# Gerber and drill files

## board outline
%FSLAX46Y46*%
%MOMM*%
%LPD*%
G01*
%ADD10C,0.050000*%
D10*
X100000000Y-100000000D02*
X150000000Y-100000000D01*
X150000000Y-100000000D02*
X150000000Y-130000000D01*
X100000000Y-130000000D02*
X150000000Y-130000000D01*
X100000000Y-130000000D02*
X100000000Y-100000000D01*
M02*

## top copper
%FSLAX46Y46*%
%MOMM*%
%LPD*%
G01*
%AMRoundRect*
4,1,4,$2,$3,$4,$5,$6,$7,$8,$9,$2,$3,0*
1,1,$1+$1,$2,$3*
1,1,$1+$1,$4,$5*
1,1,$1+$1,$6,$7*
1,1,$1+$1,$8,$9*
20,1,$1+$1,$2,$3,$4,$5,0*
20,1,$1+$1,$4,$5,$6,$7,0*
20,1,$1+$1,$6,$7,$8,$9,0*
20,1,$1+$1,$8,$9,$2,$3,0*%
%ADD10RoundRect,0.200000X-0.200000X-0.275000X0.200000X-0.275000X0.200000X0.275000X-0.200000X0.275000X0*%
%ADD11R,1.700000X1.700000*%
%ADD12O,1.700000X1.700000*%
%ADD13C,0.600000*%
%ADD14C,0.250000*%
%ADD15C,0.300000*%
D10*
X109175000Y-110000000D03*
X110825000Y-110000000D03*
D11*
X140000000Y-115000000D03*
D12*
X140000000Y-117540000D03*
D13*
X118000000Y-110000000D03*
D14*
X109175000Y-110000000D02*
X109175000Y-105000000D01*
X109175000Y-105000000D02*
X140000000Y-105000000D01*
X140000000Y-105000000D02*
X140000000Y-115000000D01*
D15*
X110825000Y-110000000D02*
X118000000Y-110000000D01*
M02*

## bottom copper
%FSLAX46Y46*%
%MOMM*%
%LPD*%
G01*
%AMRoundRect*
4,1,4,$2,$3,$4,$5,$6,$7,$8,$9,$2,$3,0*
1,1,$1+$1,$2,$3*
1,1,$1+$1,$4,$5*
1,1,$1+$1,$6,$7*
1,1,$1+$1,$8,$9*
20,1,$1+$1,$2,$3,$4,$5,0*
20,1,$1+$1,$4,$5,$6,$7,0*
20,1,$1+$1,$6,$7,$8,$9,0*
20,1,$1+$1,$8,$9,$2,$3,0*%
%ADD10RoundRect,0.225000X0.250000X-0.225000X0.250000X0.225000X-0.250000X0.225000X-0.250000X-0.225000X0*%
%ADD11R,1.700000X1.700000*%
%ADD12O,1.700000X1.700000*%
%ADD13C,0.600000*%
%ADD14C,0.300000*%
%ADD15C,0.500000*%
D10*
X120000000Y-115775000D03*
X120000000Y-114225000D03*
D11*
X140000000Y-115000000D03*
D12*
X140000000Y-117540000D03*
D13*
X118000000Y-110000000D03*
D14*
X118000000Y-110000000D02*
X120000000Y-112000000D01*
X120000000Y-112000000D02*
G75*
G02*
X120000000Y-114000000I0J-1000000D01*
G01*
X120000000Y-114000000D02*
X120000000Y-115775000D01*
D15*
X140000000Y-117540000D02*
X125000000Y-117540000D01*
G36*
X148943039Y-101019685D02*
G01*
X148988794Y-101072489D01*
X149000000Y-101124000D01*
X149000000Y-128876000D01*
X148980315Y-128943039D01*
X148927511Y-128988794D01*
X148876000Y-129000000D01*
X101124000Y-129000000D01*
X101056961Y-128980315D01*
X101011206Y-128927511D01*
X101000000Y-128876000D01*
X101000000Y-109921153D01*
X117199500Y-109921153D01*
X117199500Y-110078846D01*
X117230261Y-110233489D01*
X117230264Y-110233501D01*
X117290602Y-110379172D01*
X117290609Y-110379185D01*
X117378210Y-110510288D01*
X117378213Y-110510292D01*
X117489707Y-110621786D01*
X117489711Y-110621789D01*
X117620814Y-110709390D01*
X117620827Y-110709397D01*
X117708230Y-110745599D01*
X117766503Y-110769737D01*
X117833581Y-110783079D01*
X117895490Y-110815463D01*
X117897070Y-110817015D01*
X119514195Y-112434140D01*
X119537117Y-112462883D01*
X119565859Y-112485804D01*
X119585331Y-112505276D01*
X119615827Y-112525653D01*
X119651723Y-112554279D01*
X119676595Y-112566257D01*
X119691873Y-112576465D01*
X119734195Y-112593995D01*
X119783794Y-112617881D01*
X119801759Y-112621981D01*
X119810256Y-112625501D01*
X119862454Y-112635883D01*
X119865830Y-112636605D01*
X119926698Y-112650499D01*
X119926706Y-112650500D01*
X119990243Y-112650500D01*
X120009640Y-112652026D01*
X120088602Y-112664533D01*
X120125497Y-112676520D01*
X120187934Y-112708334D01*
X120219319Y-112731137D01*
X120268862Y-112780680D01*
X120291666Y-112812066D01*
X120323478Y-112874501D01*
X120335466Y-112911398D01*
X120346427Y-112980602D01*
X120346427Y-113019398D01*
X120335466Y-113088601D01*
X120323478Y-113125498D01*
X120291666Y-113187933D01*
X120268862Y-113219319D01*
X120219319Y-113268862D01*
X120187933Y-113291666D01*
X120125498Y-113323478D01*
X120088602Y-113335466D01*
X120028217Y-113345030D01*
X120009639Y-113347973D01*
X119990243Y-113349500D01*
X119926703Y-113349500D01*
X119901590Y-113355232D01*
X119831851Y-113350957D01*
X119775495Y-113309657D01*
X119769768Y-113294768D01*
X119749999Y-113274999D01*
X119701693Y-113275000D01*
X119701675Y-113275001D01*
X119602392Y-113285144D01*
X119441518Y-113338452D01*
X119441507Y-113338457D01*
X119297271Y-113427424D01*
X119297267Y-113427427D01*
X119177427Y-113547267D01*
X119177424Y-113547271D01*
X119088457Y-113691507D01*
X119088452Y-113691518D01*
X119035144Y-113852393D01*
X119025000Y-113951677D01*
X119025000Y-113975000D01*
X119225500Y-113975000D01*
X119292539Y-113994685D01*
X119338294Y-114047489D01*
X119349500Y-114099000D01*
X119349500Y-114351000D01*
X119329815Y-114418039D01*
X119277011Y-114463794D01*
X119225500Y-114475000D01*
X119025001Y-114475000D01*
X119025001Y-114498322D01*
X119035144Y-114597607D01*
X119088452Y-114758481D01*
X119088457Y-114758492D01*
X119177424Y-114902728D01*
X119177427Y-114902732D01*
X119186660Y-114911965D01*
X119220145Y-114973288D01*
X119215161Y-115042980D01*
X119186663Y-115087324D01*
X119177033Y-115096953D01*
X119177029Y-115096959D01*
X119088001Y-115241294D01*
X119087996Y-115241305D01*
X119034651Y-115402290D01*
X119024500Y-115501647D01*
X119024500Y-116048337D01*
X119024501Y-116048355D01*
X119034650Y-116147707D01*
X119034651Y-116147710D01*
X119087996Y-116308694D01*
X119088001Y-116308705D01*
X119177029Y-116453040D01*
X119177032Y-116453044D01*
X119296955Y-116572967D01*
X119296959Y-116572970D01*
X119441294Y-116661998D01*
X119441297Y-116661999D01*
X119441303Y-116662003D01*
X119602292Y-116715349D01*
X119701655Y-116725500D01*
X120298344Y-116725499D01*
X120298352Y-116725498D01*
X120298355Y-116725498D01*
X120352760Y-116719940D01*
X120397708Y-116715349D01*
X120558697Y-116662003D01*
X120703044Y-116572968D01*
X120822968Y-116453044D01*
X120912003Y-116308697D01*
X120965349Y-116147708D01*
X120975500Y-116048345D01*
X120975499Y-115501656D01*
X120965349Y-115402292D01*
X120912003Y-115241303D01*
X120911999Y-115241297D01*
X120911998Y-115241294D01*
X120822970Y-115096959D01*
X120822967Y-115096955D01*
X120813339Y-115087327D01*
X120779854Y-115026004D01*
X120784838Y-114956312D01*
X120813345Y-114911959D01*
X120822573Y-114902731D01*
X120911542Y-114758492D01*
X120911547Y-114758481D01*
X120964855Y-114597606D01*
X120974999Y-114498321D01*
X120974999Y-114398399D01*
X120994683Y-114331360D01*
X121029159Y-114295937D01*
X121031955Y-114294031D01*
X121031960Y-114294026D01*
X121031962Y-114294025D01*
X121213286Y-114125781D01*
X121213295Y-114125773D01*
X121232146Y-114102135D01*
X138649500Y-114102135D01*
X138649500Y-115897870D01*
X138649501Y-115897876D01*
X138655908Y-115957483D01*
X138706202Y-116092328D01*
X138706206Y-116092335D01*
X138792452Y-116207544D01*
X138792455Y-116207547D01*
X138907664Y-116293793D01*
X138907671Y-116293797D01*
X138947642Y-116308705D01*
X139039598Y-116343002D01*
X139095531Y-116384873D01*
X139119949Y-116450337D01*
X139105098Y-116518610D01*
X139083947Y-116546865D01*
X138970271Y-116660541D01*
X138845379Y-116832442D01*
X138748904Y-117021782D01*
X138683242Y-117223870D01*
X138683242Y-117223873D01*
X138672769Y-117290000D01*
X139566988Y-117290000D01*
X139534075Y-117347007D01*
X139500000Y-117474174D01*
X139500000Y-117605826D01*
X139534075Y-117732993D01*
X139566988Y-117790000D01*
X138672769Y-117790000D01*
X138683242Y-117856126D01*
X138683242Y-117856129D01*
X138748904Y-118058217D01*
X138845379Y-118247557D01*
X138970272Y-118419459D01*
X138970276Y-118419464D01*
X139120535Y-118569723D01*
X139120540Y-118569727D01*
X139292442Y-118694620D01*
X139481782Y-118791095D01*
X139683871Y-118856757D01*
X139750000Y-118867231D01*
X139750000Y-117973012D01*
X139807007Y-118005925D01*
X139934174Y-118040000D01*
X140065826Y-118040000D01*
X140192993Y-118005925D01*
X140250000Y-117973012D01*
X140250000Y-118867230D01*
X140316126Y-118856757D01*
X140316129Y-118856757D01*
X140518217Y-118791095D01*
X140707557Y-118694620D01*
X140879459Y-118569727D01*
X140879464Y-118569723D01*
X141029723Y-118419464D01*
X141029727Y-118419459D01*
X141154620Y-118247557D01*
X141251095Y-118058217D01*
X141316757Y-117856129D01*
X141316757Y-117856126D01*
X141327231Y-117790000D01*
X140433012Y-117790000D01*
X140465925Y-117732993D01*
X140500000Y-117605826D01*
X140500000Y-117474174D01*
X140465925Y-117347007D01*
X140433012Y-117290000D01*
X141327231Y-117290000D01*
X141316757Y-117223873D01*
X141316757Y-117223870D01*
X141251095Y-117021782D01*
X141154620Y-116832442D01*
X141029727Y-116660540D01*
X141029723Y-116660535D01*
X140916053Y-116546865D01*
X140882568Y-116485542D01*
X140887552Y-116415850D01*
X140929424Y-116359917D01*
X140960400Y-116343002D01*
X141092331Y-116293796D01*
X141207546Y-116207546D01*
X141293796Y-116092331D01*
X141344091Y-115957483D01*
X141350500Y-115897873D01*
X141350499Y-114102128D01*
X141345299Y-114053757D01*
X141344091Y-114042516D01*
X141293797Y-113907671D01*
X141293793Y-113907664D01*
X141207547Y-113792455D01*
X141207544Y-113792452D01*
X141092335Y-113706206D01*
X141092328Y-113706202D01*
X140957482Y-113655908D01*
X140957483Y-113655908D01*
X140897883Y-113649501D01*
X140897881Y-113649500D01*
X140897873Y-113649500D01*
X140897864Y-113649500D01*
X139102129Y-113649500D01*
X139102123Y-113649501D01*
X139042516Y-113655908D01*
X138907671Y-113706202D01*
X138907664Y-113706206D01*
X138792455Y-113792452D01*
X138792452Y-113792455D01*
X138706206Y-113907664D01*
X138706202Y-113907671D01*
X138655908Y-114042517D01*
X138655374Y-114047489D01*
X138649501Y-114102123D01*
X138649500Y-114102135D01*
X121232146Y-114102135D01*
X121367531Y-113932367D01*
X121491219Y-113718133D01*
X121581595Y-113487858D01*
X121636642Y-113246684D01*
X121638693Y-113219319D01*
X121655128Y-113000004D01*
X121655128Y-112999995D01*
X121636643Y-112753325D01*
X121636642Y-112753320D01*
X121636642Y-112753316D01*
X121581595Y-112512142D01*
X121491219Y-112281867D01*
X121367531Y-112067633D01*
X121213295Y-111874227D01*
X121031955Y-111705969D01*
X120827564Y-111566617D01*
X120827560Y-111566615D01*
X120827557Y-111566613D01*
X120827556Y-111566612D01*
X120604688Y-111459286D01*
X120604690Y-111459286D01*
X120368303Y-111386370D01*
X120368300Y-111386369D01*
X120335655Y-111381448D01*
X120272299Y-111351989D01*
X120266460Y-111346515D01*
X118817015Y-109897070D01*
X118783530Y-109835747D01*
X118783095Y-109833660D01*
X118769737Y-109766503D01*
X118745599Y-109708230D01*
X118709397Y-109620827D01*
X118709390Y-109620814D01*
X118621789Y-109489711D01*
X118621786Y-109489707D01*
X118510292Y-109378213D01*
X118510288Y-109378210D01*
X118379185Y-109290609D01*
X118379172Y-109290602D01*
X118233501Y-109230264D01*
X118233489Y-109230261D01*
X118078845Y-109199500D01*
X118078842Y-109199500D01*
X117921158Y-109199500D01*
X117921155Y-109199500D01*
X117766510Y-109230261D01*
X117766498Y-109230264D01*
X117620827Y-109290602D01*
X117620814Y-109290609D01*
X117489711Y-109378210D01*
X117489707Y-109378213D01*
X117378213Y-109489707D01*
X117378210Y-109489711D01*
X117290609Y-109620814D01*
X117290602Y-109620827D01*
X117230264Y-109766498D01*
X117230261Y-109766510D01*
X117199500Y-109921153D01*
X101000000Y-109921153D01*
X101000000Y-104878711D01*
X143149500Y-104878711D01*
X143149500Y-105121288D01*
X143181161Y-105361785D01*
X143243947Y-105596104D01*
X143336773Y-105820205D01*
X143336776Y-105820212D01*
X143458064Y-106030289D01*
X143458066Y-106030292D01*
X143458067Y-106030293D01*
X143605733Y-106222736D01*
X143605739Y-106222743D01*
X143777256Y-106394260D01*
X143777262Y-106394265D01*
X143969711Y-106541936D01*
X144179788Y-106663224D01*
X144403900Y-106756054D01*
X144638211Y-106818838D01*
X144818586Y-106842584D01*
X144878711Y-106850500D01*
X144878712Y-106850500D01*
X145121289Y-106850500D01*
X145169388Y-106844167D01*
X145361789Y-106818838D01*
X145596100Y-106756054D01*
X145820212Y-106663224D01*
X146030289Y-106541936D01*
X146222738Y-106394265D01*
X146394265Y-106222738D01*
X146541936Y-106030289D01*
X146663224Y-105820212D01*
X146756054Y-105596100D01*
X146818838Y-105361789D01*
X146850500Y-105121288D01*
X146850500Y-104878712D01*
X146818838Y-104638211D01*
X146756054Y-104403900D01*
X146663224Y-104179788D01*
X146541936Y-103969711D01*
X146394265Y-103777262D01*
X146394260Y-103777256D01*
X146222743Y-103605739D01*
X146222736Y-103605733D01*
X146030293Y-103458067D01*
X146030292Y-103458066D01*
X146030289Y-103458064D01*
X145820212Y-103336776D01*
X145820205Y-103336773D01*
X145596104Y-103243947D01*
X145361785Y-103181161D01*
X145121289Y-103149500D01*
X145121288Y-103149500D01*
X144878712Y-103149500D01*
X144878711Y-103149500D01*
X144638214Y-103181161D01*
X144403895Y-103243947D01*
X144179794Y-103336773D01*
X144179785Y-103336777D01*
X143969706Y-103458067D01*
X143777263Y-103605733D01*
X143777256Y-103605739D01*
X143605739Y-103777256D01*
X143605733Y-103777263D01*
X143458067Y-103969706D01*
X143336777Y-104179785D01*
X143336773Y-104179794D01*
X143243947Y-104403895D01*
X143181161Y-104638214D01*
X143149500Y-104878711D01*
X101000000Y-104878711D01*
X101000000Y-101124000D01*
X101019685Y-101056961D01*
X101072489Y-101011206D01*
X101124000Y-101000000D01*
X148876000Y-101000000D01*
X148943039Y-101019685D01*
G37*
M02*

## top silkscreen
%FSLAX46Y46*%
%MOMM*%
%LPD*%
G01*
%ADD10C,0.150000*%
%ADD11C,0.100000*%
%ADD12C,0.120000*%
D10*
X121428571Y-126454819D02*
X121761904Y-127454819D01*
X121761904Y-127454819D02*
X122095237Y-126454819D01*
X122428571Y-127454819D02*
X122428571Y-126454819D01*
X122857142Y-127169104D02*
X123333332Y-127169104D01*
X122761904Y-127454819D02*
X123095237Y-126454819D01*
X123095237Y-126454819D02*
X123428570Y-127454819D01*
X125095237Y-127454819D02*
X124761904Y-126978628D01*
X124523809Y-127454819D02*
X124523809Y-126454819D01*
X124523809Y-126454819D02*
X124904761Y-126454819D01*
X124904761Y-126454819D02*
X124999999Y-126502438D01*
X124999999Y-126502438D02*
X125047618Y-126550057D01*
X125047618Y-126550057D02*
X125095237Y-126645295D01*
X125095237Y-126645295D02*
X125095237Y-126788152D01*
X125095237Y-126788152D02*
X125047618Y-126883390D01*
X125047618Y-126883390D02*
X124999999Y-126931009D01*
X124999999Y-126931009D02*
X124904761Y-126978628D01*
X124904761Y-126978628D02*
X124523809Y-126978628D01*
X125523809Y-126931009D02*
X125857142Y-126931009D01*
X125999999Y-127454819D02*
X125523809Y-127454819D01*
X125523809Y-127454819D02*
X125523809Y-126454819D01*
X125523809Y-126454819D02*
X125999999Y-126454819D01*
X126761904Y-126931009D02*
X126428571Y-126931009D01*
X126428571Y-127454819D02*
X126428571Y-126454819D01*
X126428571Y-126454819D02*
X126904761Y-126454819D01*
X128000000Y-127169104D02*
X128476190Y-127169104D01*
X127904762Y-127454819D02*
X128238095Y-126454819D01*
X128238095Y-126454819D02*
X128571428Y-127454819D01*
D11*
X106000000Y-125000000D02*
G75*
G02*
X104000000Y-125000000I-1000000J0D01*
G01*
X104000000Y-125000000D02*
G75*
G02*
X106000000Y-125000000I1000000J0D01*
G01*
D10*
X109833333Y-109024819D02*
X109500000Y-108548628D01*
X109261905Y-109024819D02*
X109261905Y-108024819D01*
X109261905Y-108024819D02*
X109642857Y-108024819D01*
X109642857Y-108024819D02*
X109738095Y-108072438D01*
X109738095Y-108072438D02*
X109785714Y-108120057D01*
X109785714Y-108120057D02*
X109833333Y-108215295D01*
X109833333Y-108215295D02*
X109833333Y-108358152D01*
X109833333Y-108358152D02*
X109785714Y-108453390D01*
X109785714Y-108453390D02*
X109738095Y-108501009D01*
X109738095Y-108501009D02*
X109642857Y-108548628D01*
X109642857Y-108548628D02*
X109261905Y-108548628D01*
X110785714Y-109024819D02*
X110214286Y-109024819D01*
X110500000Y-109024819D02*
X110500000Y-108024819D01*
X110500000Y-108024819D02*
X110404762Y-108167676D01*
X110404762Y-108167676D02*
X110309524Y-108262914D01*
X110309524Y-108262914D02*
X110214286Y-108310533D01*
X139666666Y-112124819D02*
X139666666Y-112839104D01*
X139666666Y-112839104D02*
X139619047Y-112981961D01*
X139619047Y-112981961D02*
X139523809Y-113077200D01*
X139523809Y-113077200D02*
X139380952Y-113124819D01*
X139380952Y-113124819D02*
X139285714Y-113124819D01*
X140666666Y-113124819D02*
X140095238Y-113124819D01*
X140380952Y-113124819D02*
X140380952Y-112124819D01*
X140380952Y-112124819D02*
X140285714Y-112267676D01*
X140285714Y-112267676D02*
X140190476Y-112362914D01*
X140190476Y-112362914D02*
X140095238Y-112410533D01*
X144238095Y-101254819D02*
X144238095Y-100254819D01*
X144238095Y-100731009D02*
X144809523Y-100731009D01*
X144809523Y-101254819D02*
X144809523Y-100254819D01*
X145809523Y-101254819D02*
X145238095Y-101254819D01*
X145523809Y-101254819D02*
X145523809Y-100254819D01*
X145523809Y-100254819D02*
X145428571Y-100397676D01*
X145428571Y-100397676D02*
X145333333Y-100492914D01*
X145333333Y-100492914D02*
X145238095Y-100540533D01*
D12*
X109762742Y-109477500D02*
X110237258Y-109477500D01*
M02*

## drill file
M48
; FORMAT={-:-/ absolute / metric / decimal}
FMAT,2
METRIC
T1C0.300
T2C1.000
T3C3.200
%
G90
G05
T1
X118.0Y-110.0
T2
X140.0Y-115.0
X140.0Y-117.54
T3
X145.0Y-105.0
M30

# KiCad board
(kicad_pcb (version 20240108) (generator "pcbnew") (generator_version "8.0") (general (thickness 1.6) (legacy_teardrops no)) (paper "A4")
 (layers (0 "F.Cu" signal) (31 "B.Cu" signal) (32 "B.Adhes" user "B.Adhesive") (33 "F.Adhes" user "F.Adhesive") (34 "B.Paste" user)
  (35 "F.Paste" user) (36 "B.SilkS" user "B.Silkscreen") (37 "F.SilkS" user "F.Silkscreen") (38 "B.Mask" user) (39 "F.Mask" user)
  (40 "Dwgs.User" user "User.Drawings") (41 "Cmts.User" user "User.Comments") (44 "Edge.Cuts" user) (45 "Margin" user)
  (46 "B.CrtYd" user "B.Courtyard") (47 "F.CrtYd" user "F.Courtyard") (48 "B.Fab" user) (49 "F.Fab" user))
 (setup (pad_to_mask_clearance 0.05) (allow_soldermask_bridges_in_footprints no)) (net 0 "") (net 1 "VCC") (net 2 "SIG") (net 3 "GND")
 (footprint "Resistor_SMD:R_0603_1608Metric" (layer "F.Cu") (at 110 110)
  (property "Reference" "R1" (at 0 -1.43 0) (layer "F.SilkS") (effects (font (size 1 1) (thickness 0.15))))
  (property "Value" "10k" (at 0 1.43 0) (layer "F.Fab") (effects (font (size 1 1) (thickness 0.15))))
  (fp_line (start -0.237258 -0.5225) (end 0.237258 -0.5225) (stroke (width 0.12) (type solid)) (layer "F.SilkS"))
  (pad "1" smd roundrect (at -0.825 0) (size 0.8 0.95) (layers "F.Cu" "F.Paste" "F.Mask") (roundrect_rratio 0.25) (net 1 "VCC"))
  (pad "2" smd roundrect (at 0.825 0) (size 0.8 0.95) (layers "F.Cu" "F.Paste" "F.Mask") (roundrect_rratio 0.25) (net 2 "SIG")))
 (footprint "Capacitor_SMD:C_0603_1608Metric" (layer "B.Cu") (at 120 115 90)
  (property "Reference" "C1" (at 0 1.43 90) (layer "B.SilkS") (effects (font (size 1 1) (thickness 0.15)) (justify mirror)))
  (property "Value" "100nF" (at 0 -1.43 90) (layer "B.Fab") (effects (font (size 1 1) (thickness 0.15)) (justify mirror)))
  (pad "1" smd roundrect (at -0.775 0 90) (size 0.9 0.95) (layers "B.Cu" "B.Paste" "B.Mask") (roundrect_rratio 0.25) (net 2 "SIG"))
  (pad "2" smd roundrect (at 0.775 0 90) (size 0.9 0.95) (layers "B.Cu" "B.Paste" "B.Mask") (roundrect_rratio 0.25) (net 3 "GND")))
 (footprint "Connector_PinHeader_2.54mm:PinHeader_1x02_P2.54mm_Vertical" (layer "F.Cu") (at 140 115)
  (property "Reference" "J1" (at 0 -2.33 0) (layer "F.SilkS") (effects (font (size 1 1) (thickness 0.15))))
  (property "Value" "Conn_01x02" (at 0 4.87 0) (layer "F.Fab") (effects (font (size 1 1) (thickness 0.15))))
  (pad "1" thru_hole rect (at 0 0) (size 1.7 1.7) (drill 1) (layers "*.Cu" "*.Mask") (remove_unused_layers no) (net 1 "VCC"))
  (pad "2" thru_hole oval (at 0 2.54) (size 1.7 1.7) (drill 1) (layers "*.Cu" "*.Mask") (remove_unused_layers no) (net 3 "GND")))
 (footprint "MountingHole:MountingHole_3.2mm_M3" (layer "F.Cu") (at 145 105)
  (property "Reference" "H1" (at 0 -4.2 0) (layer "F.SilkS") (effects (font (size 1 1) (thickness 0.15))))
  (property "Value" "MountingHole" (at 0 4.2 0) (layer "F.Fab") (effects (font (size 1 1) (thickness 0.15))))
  (pad "" np_thru_hole circle (at 0 0) (size 3.2 3.2) (drill 3.2) (layers "*.Cu" "*.Mask")))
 (gr_line (start 100 100) (end 150 100) (stroke (width 0.05) (type default)) (layer "Edge.Cuts"))
 (gr_line (start 150 100) (end 150 130) (stroke (width 0.05) (type default)) (layer "Edge.Cuts"))
 (gr_line (start 100 130) (end 150 130) (stroke (width 0.05) (type default)) (layer "Edge.Cuts"))
 (gr_line (start 100 130) (end 100 100) (stroke (width 0.05) (type default)) (layer "Edge.Cuts"))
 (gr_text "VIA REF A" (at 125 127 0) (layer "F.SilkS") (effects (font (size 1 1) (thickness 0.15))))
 (gr_circle (center 105 125) (end 106 125) (stroke (width 0.1) (type default)) (fill none) (layer "F.SilkS"))
 (segment (start 109.175 110) (end 109.175 105) (width 0.25) (layer "F.Cu") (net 1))
 (segment (start 109.175 105) (end 140 105) (width 0.25) (layer "F.Cu") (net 1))
 (segment (start 140 105) (end 140 115) (width 0.25) (layer "F.Cu") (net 1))
 (segment (start 110.825 110) (end 118 110) (width 0.3) (layer "F.Cu") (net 2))
 (via (at 118 110) (size 0.6) (drill 0.3) (layers "F.Cu" "B.Cu") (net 2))
 (segment (start 118 110) (end 120 112) (width 0.3) (layer "B.Cu") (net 2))
 (arc (start 120 112) (mid 121 113) (end 120 114) (width 0.3) (layer "B.Cu") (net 2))
 (segment (start 120 114) (end 120 115.775) (width 0.3) (layer "B.Cu") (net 2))
 (segment (start 140 117.54) (end 125 117.54) (width 0.5) (layer "B.Cu") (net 3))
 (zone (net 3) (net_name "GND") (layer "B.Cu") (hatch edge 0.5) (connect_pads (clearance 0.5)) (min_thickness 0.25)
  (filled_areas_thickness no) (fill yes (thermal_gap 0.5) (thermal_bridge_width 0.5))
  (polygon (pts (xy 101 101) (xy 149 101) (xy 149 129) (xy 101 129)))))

